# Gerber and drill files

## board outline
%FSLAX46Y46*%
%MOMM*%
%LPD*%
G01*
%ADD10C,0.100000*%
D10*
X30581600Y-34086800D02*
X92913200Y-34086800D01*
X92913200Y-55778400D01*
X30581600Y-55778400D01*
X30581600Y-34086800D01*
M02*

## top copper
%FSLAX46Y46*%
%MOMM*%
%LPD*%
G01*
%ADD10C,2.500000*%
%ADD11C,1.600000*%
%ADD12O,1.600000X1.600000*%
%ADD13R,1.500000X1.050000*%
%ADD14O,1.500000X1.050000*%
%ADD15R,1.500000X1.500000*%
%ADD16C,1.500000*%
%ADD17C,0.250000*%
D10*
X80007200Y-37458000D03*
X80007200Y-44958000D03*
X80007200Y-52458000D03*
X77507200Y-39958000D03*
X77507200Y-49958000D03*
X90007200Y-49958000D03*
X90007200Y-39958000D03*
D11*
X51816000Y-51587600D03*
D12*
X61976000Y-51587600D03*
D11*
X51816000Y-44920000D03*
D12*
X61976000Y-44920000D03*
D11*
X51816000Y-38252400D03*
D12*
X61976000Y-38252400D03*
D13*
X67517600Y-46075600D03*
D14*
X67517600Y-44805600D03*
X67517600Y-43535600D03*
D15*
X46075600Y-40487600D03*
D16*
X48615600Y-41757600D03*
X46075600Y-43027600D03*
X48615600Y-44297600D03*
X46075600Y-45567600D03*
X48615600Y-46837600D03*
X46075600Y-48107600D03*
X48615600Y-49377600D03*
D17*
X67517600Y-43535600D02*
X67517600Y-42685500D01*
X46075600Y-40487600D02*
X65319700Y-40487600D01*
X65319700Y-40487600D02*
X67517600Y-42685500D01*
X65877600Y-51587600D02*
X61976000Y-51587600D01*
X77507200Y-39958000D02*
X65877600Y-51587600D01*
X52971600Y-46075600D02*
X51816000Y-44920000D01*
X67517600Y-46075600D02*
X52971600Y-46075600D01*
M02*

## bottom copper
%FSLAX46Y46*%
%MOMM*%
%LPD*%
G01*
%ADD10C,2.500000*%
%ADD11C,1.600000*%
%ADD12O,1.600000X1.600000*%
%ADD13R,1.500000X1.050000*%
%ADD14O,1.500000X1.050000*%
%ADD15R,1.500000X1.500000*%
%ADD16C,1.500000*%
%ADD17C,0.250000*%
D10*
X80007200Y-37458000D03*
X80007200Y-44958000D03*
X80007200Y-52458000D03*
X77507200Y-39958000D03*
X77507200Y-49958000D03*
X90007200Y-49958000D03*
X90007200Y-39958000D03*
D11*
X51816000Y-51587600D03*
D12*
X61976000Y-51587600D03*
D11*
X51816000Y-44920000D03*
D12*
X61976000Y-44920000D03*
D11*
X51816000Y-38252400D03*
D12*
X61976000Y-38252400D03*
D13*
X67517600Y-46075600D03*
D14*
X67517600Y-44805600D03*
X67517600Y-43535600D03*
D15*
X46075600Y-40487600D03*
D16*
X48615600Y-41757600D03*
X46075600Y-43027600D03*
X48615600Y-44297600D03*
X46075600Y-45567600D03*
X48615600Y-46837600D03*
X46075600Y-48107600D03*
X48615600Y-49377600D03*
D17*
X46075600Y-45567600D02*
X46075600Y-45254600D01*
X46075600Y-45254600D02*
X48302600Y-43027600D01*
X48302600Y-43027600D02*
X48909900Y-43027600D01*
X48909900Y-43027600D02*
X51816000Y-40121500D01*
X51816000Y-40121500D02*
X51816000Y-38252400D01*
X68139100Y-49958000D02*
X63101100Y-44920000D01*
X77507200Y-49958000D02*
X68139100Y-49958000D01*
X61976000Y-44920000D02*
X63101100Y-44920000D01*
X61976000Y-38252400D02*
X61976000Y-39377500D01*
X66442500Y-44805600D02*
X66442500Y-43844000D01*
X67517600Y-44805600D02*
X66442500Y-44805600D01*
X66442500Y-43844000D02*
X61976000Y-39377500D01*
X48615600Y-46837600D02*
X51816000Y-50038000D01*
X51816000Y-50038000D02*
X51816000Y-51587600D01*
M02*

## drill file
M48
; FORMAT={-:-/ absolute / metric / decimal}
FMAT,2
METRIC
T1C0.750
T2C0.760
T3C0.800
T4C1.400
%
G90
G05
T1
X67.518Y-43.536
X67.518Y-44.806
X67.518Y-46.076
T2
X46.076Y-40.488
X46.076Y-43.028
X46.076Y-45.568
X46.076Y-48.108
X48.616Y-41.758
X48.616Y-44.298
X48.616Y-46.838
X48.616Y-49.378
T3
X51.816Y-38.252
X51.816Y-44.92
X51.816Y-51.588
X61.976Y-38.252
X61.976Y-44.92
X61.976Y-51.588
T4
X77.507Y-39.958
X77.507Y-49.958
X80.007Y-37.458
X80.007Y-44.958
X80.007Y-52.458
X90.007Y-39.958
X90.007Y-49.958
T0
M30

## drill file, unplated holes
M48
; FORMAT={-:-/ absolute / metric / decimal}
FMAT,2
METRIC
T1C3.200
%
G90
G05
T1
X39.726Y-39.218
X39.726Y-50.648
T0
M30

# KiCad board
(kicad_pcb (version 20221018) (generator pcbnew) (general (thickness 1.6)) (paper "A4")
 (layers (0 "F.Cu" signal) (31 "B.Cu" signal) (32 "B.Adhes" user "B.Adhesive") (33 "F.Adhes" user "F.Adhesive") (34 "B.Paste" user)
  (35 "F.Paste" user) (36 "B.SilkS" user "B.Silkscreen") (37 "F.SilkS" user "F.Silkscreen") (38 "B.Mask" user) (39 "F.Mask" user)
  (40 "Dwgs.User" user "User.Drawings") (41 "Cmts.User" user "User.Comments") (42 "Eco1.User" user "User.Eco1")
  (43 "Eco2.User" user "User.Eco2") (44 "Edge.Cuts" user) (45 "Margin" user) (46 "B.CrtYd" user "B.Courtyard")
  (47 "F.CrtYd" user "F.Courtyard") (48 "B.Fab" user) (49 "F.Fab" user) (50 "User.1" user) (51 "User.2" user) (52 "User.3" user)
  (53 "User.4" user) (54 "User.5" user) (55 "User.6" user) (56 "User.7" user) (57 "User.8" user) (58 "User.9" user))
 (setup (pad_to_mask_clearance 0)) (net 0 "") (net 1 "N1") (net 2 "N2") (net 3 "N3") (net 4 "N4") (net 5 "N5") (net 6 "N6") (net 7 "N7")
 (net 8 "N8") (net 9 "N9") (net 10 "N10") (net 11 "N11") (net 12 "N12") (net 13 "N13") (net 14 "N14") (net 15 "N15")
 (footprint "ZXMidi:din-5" (layer "F.Cu") (at 83.0072 44.958 90)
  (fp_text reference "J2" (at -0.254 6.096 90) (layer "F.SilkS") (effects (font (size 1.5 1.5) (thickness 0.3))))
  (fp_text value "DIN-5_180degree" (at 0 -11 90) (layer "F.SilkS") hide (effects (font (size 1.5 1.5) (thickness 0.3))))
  (pad "1" thru_hole circle (at 7.5 -3 90) (size 2.5 2.5) (drill 1.4) (layers "*.Cu" "*.Mask") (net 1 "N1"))
  (pad "2" thru_hole circle (at 0 -3 90) (size 2.5 2.5) (drill 1.4) (layers "*.Cu" "*.Mask") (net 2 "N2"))
  (pad "3" thru_hole circle (at -7.5 -3 90) (size 2.5 2.5) (drill 1.4) (layers "*.Cu" "*.Mask") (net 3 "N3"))
  (pad "4" thru_hole circle (at 5 -5.5 90) (size 2.5 2.5) (drill 1.4) (layers "*.Cu" "*.Mask") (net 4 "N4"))
  (pad "5" thru_hole circle (at -5 -5.5 90) (size 2.5 2.5) (drill 1.4) (layers "*.Cu" "*.Mask") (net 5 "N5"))
  (pad "6" thru_hole circle (at -5 7 90) (size 2.5 2.5) (drill 1.4) (layers "*.Cu" "*.Mask"))
  (pad "6" thru_hole circle (at 5 7 90) (size 2.5 2.5) (drill 1.4) (layers "*.Cu" "*.Mask")))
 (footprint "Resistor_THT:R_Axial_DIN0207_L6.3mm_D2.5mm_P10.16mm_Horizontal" (layer "F.Cu") (at 51.816 51.5876)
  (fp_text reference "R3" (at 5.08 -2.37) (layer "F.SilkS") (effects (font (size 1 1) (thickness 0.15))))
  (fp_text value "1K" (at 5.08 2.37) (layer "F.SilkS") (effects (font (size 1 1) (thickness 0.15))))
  (pad "1" thru_hole circle (at 0 0) (size 1.6 1.6) (drill 0.8) (layers "*.Cu" "*.Mask") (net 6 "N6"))
  (pad "2" thru_hole oval (at 10.16 0) (size 1.6 1.6) (drill 0.8) (layers "*.Cu" "*.Mask") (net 4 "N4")))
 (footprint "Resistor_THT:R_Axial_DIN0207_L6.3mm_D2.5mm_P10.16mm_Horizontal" (layer "F.Cu") (at 51.816 44.92)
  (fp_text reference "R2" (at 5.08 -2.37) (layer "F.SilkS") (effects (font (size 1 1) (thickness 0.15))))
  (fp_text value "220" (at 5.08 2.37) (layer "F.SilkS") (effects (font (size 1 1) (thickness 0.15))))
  (pad "1" thru_hole circle (at 0 0) (size 1.6 1.6) (drill 0.8) (layers "*.Cu" "*.Mask") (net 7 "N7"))
  (pad "2" thru_hole oval (at 10.16 0) (size 1.6 1.6) (drill 0.8) (layers "*.Cu" "*.Mask") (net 5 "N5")))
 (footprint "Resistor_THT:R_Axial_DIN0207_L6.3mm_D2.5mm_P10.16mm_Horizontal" (layer "F.Cu") (at 51.816 38.2524)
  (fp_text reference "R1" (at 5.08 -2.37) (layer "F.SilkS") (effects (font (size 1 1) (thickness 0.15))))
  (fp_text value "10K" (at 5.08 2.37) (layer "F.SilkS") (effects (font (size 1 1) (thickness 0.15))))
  (pad "1" thru_hole circle (at 0 0) (size 1.6 1.6) (drill 0.8) (layers "*.Cu" "*.Mask") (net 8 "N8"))
  (pad "2" thru_hole oval (at 10.16 0) (size 1.6 1.6) (drill 0.8) (layers "*.Cu" "*.Mask") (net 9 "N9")))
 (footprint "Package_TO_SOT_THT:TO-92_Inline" (layer "F.Cu") (at 67.5176 46.0756 90)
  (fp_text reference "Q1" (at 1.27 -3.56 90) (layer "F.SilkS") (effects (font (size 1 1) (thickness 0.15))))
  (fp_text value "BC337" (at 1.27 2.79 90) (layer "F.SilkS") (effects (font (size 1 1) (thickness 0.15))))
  (pad "1" thru_hole rect (at 0 0 90) (size 1.05 1.5) (drill 0.75) (layers "*.Cu" "*.Mask") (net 7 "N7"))
  (pad "2" thru_hole oval (at 1.27 0 90) (size 1.05 1.5) (drill 0.75) (layers "*.Cu" "*.Mask") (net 9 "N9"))
  (pad "3" thru_hole oval (at 2.54 0 90) (size 1.05 1.5) (drill 0.75) (layers "*.Cu" "*.Mask") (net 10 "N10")))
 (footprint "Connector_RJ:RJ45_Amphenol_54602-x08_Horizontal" (layer "F.Cu") (at 46.0756 40.4876 -90)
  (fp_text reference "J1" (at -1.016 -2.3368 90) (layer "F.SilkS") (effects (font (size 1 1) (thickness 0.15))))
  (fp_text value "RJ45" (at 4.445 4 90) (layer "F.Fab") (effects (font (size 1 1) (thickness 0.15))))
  (pad "" np_thru_hole circle (at -1.27 6.35 270) (size 3.2 3.2) (drill 3.2) (layers "*.Cu" "*.Mask"))
  (pad "" np_thru_hole circle (at 10.16 6.35 270) (size 3.2 3.2) (drill 3.2) (layers "*.Cu" "*.Mask"))
  (pad "1" thru_hole rect (at 0 0 270) (size 1.5 1.5) (drill 0.76) (layers "*.Cu" "*.Mask") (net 10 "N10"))
  (pad "2" thru_hole circle (at 1.27 -2.54 270) (size 1.5 1.5) (drill 0.76) (layers "*.Cu" "*.Mask") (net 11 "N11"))
  (pad "3" thru_hole circle (at 2.54 0 270) (size 1.5 1.5) (drill 0.76) (layers "*.Cu" "*.Mask") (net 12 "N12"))
  (pad "4" thru_hole circle (at 3.81 -2.54 270) (size 1.5 1.5) (drill 0.76) (layers "*.Cu" "*.Mask") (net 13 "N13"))
  (pad "5" thru_hole circle (at 5.08 0 270) (size 1.5 1.5) (drill 0.76) (layers "*.Cu" "*.Mask") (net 8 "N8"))
  (pad "6" thru_hole circle (at 6.35 -2.54 270) (size 1.5 1.5) (drill 0.76) (layers "*.Cu" "*.Mask") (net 6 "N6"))
  (pad "7" thru_hole circle (at 7.62 0 270) (size 1.5 1.5) (drill 0.76) (layers "*.Cu" "*.Mask") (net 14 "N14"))
  (pad "8" thru_hole circle (at 8.89 -2.54 270) (size 1.5 1.5) (drill 0.76) (layers "*.Cu" "*.Mask") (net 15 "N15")))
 (gr_rect (start 30.5816 34.0868) (end 92.9132 55.7784) (stroke (width 0.1) (type default)) (fill none) (layer "Edge.Cuts"))
 (segment (start 67.5176 43.5356) (end 67.5176 42.6855) (width 0.25) (layer "F.Cu") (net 10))
 (segment (start 46.0756 40.4876) (end 65.3197 40.4876) (width 0.25) (layer "F.Cu") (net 10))
 (segment (start 65.3197 40.4876) (end 67.5176 42.6855) (width 0.25) (layer "F.Cu") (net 10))
 (segment (start 46.0756 45.5676) (end 46.0756 45.2546) (width 0.25) (layer "B.Cu") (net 8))
 (segment (start 46.0756 45.2546) (end 48.3026 43.0276) (width 0.25) (layer "B.Cu") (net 8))
 (segment (start 48.3026 43.0276) (end 48.9099 43.0276) (width 0.25) (layer "B.Cu") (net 8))
 (segment (start 48.9099 43.0276) (end 51.816 40.1215) (width 0.25) (layer "B.Cu") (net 8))
 (segment (start 51.816 40.1215) (end 51.816 38.2524) (width 0.25) (layer "B.Cu") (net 8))
 (segment (start 65.8776 51.5876) (end 61.976 51.5876) (width 0.25) (layer "F.Cu") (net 4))
 (segment (start 77.5072 39.958) (end 65.8776 51.5876) (width 0.25) (layer "F.Cu") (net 4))
 (segment (start 68.1391 49.958) (end 63.1011 44.92) (width 0.25) (layer "B.Cu") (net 5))
 (segment (start 77.5072 49.958) (end 68.1391 49.958) (width 0.25) (layer "B.Cu") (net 5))
 (segment (start 61.976 44.92) (end 63.1011 44.92) (width 0.25) (layer "B.Cu") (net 5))
 (segment (start 52.9716 46.0756) (end 51.816 44.92) (width 0.25) (layer "F.Cu") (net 7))
 (segment (start 67.5176 46.0756) (end 52.9716 46.0756) (width 0.25) (layer "F.Cu") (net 7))
 (segment (start 61.976 38.2524) (end 61.976 39.3775) (width 0.25) (layer "B.Cu") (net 9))
 (segment (start 66.4425 44.8056) (end 66.4425 43.844) (width 0.25) (layer "B.Cu") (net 9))
 (segment (start 67.5176 44.8056) (end 66.4425 44.8056) (width 0.25) (layer "B.Cu") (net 9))
 (segment (start 66.4425 43.844) (end 61.976 39.3775) (width 0.25) (layer "B.Cu") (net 9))
 (segment (start 48.6156 46.8376) (end 51.816 50.038) (width 0.25) (layer "B.Cu") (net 6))
 (segment (start 51.816 50.038) (end 51.816 51.5876) (width 0.25) (layer "B.Cu") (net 6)))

